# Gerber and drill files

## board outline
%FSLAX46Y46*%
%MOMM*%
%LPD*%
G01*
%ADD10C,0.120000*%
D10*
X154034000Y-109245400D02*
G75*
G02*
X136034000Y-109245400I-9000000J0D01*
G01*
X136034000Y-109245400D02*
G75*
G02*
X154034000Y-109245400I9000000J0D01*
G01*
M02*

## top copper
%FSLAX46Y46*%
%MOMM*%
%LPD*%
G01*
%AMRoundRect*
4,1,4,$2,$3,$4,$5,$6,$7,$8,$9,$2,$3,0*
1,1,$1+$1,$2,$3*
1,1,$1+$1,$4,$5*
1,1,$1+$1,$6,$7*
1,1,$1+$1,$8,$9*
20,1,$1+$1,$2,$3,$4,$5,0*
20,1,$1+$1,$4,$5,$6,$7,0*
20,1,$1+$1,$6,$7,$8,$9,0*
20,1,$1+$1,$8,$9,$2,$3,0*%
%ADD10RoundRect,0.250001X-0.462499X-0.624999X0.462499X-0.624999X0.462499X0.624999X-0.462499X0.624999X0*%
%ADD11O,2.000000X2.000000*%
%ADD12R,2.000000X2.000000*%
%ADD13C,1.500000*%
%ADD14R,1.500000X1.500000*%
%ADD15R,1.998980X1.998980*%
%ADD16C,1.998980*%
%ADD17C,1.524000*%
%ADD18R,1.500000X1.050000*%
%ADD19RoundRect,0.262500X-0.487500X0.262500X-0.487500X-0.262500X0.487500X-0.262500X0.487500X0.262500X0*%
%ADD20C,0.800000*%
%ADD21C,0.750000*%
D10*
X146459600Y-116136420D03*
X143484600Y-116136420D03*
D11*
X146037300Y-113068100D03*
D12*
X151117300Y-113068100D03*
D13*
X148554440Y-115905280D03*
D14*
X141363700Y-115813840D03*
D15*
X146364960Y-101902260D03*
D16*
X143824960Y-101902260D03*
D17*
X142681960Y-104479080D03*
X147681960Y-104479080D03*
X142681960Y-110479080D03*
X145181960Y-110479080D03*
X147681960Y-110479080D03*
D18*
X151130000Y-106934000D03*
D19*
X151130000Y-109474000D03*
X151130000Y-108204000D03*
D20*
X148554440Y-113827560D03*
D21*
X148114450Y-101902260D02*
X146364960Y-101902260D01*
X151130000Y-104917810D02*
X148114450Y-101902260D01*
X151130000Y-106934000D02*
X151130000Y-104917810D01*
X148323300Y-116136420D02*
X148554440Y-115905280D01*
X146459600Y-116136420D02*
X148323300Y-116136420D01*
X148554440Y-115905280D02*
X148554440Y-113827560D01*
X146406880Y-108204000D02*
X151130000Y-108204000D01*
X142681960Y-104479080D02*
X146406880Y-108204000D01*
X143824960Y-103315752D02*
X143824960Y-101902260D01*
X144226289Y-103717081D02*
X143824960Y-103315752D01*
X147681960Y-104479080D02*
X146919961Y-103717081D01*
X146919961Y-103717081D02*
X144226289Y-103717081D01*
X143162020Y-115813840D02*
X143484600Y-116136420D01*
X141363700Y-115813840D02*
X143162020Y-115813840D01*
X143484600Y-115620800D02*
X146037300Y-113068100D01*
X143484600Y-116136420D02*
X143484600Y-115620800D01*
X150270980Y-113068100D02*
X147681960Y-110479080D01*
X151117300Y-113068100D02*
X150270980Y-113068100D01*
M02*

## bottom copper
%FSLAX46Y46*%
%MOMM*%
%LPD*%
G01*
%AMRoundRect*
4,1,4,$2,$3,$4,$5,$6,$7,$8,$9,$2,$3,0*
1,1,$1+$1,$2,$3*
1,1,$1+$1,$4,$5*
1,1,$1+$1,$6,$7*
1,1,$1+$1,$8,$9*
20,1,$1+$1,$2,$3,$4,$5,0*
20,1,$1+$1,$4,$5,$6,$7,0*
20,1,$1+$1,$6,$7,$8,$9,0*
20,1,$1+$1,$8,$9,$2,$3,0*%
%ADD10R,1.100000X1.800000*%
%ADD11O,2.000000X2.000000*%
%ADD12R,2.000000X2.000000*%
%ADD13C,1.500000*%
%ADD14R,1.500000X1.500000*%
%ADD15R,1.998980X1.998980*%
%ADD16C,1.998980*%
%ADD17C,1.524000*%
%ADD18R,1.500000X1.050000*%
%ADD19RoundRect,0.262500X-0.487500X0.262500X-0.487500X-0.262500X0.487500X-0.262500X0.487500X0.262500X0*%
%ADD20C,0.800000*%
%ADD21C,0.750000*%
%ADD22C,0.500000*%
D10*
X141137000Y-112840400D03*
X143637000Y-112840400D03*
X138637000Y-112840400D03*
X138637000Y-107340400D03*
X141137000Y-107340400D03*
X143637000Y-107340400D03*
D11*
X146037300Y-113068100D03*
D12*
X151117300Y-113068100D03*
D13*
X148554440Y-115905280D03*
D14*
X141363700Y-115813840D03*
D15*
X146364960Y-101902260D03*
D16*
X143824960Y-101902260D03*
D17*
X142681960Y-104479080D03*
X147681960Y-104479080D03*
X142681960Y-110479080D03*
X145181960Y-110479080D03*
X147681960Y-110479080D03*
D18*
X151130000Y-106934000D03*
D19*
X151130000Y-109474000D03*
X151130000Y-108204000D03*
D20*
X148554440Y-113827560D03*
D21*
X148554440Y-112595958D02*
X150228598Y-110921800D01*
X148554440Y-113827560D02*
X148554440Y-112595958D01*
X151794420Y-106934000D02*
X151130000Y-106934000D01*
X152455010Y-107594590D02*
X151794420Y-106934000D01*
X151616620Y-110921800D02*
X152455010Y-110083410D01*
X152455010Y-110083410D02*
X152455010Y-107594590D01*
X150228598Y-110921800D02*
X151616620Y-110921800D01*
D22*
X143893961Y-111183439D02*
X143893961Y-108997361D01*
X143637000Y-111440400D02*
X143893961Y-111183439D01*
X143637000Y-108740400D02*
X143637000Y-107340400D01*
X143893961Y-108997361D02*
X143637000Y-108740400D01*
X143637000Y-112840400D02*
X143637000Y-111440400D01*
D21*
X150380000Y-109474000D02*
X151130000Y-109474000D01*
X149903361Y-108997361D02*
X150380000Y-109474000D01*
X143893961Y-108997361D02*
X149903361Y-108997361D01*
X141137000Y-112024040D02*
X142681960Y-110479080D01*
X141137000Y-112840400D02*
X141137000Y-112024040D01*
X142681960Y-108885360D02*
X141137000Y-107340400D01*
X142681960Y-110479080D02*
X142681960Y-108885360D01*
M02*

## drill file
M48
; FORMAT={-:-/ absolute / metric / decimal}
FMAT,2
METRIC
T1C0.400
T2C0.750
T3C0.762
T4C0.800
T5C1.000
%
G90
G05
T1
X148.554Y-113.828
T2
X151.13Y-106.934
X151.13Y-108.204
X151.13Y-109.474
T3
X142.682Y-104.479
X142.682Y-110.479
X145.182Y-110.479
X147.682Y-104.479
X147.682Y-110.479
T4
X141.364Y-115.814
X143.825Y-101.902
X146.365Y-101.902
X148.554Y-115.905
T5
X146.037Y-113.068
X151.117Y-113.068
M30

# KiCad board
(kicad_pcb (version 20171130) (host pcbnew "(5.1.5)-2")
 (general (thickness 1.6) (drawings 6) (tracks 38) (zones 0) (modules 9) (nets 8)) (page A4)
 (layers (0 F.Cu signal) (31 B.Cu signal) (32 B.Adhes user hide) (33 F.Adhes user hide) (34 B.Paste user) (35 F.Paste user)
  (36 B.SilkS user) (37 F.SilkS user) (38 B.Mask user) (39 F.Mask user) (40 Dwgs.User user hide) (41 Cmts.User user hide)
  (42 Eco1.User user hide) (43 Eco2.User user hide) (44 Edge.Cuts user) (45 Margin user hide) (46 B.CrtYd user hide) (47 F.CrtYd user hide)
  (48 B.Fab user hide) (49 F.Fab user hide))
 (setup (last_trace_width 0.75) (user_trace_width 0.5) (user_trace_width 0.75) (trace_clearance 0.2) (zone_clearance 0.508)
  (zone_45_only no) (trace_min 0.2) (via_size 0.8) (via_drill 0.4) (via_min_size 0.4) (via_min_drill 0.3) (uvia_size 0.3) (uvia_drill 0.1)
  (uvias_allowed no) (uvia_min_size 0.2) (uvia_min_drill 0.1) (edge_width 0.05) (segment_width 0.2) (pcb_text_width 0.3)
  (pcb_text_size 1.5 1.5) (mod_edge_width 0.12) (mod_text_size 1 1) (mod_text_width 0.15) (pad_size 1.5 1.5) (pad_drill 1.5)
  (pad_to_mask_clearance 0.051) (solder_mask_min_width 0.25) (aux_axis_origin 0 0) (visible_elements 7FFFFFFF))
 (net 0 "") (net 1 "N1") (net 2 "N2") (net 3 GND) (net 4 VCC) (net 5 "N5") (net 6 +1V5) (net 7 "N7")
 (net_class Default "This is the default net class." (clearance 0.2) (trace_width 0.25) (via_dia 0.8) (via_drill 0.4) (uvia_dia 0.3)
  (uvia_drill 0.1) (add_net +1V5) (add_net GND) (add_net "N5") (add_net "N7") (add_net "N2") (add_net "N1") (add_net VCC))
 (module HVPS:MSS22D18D (layer B.Cu) (at 140.4874 104.902 180)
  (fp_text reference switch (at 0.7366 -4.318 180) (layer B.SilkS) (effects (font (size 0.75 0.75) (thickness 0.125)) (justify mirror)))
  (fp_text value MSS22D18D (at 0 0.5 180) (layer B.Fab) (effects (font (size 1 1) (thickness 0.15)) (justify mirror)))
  (pad 2 smd rect (at -0.6496 -7.9384 180) (size 1.1 1.8) (layers B.Cu B.Paste B.Mask) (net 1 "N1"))
  (pad 1 smd rect (at -3.1496 -7.9384 180) (size 1.1 1.8) (layers B.Cu B.Paste B.Mask) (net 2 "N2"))
  (pad 3 smd rect (at 1.8504 -7.9384 180) (size 1.1 1.8) (layers B.Cu B.Paste B.Mask))
  (pad 3 smd rect (at 1.8504 -2.4384 180) (size 1.1 1.8) (layers B.Cu B.Paste B.Mask))
  (pad 2 smd rect (at -0.6496 -2.4384 180) (size 1.1 1.8) (layers B.Cu B.Paste B.Mask) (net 1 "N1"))
  (pad 1 smd rect (at -3.1496 -2.4384 180) (size 1.1 1.8) (layers B.Cu B.Paste B.Mask) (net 2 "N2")))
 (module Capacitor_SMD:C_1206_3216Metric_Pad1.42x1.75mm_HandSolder (layer F.Cu) (at 144.9721 116.13642)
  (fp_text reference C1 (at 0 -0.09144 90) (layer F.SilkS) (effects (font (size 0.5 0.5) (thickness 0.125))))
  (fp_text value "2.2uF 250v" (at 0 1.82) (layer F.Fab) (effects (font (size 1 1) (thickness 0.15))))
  (pad 2 smd roundrect (at 1.4875 0) (size 1.425 1.75) (layers F.Cu F.Paste F.Mask) (roundrect_rratio 0.175439) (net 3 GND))
  (pad 1 smd roundrect (at -1.4875 0) (size 1.425 1.75) (layers F.Cu F.Paste F.Mask) (roundrect_rratio 0.175439) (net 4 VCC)))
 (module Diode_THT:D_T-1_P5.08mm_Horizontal (layer F.Cu) (at 151.1173 113.0681 180)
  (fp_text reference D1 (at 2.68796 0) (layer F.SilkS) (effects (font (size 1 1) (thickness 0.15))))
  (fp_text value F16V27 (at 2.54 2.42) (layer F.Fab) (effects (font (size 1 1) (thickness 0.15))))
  (pad 2 thru_hole oval (at 5.08 0 180) (size 2 2) (drill 1) (layers *.Cu *.Mask) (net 4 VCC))
  (pad 1 thru_hole rect (at 0 0 180) (size 2 2) (drill 1) (layers *.Cu *.Mask) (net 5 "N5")))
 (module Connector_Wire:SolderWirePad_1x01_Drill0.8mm (layer F.Cu) (at 148.55444 115.90528)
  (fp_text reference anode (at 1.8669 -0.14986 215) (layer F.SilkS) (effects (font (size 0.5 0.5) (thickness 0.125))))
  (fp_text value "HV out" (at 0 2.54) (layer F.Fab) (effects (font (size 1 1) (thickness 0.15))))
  (pad 1 thru_hole circle (at 0 0) (size 1.5 1.5) (drill 0.8001) (layers *.Cu *.Mask) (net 3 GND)))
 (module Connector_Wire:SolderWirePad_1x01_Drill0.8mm (layer F.Cu) (at 141.3637 115.81384)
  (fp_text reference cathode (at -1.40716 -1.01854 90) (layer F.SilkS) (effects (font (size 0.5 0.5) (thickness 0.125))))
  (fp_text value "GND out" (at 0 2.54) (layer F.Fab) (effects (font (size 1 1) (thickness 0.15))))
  (pad 1 thru_hole rect (at 0 0) (size 1.5 1.5) (drill 0.8001) (layers *.Cu *.Mask) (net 4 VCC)))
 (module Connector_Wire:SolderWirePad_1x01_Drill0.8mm (layer F.Cu) (at 146.36496 101.90226)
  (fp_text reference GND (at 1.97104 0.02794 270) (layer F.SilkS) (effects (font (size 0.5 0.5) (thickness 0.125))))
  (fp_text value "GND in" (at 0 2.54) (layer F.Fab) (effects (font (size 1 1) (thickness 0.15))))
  (pad 1 thru_hole rect (at 0 0) (size 1.99898 1.99898) (drill 0.8001) (layers *.Cu *.Mask) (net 3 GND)))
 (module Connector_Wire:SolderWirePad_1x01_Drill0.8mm (layer F.Cu) (at 143.82496 101.90226)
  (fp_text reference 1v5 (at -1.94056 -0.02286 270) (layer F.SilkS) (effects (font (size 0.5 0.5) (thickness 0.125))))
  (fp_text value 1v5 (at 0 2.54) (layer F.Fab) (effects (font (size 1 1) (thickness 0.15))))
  (pad 1 thru_hole circle (at 0 0) (size 1.99898 1.99898) (drill 0.8001) (layers *.Cu *.Mask) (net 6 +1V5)))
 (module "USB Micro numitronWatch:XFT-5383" (layer F.Cu) (at 145.51152 100.44556)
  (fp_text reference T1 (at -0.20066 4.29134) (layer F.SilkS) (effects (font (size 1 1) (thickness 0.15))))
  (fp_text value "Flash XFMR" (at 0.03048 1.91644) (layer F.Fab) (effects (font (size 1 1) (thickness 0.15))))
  (pad 2 thru_hole circle (at -2.82956 4.03352 180) (size 1.524 1.524) (drill 0.762) (layers *.Cu *.Mask) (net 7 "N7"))
  (pad 1 thru_hole circle (at 2.17044 4.03352 180) (size 1.524 1.524) (drill 0.762) (layers *.Cu *.Mask) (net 6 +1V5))
  (pad 3 thru_hole circle (at -2.82956 10.03352 180) (size 1.524 1.524) (drill 0.762) (layers *.Cu *.Mask) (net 1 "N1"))
  (pad 5 thru_hole circle (at -0.32956 10.03352 180) (size 1.524 1.524) (drill 0.762) (layers *.Cu *.Mask))
  (pad 4 thru_hole circle (at 2.17044 10.03352 180) (size 1.524 1.524) (drill 0.762) (layers *.Cu *.Mask) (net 5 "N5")))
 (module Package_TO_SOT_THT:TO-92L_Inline (layer F.Cu) (at 151.13 106.934 270)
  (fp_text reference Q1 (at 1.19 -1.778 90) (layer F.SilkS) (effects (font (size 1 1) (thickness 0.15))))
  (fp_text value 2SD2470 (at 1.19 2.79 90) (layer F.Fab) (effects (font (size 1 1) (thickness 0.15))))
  (pad 1 thru_hole rect (at 0 0 270) (size 1.05 1.5) (drill 0.75) (layers *.Cu *.Mask) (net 3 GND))
  (pad 3 thru_hole roundrect (at 2.54 0 270) (size 1.05 1.5) (drill 0.75) (layers *.Cu *.Mask) (roundrect_rratio 0.25) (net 2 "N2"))
  (pad 2 thru_hole roundrect (at 1.27 0 270) (size 1.05 1.5) (drill 0.75) (layers *.Cu *.Mask) (roundrect_rratio 0.25) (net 7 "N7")))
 (gr_circle (center 145.034 109.2454) (end 154.034 109.2454) (layer Edge.Cuts) (width 0.12))
 (segment (start 148.11445 101.90226) (end 146.36496 101.90226) (width 0.75) (layer F.Cu) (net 3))
 (segment (start 151.13 104.91781) (end 148.11445 101.90226) (width 0.75) (layer F.Cu) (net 3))
 (segment (start 151.13 106.934) (end 151.13 104.91781) (width 0.75) (layer F.Cu) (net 3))
 (segment (start 148.3233 116.13642) (end 148.55444 115.90528) (width 0.75) (layer F.Cu) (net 3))
 (segment (start 146.4596 116.13642) (end 148.3233 116.13642) (width 0.75) (layer F.Cu) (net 3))
 (segment (start 148.55444 115.90528) (end 148.55444 113.82756) (width 0.75) (layer F.Cu) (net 3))
 (via (at 148.55444 113.82756) (size 0.8) (drill 0.4) (layers F.Cu B.Cu) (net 3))
 (segment (start 148.55444 112.595958) (end 150.228598 110.9218) (width 0.75) (layer B.Cu) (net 3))
 (segment (start 148.55444 113.82756) (end 148.55444 112.595958) (width 0.75) (layer B.Cu) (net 3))
 (segment (start 151.79442 106.934) (end 151.13 106.934) (width 0.75) (layer B.Cu) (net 3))
 (segment (start 152.45501 107.59459) (end 151.79442 106.934) (width 0.75) (layer B.Cu) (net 3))
 (segment (start 151.61662 110.9218) (end 152.45501 110.08341) (width 0.75) (layer B.Cu) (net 3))
 (segment (start 152.45501 110.08341) (end 152.45501 107.59459) (width 0.75) (layer B.Cu) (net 3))
 (segment (start 150.228598 110.9218) (end 151.61662 110.9218) (width 0.75) (layer B.Cu) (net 3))
 (segment (start 143.893961 111.183439) (end 143.893961 108.997361) (width 0.5) (layer B.Cu) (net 2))
 (segment (start 143.637 111.4404) (end 143.893961 111.183439) (width 0.5) (layer B.Cu) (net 2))
 (segment (start 143.637 108.7404) (end 143.637 107.3404) (width 0.5) (layer B.Cu) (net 2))
 (segment (start 143.893961 108.997361) (end 143.637 108.7404) (width 0.5) (layer B.Cu) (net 2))
 (segment (start 143.637 112.8404) (end 143.637 111.4404) (width 0.5) (layer B.Cu) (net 2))
 (segment (start 150.38 109.474) (end 151.13 109.474) (width 0.75) (layer B.Cu) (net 2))
 (segment (start 149.903361 108.997361) (end 150.38 109.474) (width 0.75) (layer B.Cu) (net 2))
 (segment (start 143.893961 108.997361) (end 149.903361 108.997361) (width 0.75) (layer B.Cu) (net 2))
 (segment (start 146.40688 108.204) (end 151.13 108.204) (width 0.75) (layer F.Cu) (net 7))
 (segment (start 142.68196 104.47908) (end 146.40688 108.204) (width 0.75) (layer F.Cu) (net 7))
 (segment (start 143.82496 103.315752) (end 143.82496 101.90226) (width 0.75) (layer F.Cu) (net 6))
 (segment (start 144.226289 103.717081) (end 143.82496 103.315752) (width 0.75) (layer F.Cu) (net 6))
 (segment (start 147.68196 104.47908) (end 146.919961 103.717081) (width 0.75) (layer F.Cu) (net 6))
 (segment (start 146.919961 103.717081) (end 144.226289 103.717081) (width 0.75) (layer F.Cu) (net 6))
 (segment (start 143.16202 115.81384) (end 143.4846 116.13642) (width 0.75) (layer F.Cu) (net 4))
 (segment (start 141.3637 115.81384) (end 143.16202 115.81384) (width 0.75) (layer F.Cu) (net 4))
 (segment (start 143.4846 115.6208) (end 146.0373 113.0681) (width 0.75) (layer F.Cu) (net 4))
 (segment (start 143.4846 116.13642) (end 143.4846 115.6208) (width 0.75) (layer F.Cu) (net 4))
 (segment (start 150.27098 113.0681) (end 147.68196 110.47908) (width 0.75) (layer F.Cu) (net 5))
 (segment (start 151.1173 113.0681) (end 150.27098 113.0681) (width 0.75) (layer F.Cu) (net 5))
 (segment (start 141.137 112.02404) (end 142.68196 110.47908) (width 0.75) (layer B.Cu) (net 1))
 (segment (start 141.137 112.8404) (end 141.137 112.02404) (width 0.75) (layer B.Cu) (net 1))
 (segment (start 142.68196 108.88536) (end 141.137 107.3404) (width 0.75) (layer B.Cu) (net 1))
 (segment (start 142.68196 110.47908) (end 142.68196 108.88536) (width 0.75) (layer B.Cu) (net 1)))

